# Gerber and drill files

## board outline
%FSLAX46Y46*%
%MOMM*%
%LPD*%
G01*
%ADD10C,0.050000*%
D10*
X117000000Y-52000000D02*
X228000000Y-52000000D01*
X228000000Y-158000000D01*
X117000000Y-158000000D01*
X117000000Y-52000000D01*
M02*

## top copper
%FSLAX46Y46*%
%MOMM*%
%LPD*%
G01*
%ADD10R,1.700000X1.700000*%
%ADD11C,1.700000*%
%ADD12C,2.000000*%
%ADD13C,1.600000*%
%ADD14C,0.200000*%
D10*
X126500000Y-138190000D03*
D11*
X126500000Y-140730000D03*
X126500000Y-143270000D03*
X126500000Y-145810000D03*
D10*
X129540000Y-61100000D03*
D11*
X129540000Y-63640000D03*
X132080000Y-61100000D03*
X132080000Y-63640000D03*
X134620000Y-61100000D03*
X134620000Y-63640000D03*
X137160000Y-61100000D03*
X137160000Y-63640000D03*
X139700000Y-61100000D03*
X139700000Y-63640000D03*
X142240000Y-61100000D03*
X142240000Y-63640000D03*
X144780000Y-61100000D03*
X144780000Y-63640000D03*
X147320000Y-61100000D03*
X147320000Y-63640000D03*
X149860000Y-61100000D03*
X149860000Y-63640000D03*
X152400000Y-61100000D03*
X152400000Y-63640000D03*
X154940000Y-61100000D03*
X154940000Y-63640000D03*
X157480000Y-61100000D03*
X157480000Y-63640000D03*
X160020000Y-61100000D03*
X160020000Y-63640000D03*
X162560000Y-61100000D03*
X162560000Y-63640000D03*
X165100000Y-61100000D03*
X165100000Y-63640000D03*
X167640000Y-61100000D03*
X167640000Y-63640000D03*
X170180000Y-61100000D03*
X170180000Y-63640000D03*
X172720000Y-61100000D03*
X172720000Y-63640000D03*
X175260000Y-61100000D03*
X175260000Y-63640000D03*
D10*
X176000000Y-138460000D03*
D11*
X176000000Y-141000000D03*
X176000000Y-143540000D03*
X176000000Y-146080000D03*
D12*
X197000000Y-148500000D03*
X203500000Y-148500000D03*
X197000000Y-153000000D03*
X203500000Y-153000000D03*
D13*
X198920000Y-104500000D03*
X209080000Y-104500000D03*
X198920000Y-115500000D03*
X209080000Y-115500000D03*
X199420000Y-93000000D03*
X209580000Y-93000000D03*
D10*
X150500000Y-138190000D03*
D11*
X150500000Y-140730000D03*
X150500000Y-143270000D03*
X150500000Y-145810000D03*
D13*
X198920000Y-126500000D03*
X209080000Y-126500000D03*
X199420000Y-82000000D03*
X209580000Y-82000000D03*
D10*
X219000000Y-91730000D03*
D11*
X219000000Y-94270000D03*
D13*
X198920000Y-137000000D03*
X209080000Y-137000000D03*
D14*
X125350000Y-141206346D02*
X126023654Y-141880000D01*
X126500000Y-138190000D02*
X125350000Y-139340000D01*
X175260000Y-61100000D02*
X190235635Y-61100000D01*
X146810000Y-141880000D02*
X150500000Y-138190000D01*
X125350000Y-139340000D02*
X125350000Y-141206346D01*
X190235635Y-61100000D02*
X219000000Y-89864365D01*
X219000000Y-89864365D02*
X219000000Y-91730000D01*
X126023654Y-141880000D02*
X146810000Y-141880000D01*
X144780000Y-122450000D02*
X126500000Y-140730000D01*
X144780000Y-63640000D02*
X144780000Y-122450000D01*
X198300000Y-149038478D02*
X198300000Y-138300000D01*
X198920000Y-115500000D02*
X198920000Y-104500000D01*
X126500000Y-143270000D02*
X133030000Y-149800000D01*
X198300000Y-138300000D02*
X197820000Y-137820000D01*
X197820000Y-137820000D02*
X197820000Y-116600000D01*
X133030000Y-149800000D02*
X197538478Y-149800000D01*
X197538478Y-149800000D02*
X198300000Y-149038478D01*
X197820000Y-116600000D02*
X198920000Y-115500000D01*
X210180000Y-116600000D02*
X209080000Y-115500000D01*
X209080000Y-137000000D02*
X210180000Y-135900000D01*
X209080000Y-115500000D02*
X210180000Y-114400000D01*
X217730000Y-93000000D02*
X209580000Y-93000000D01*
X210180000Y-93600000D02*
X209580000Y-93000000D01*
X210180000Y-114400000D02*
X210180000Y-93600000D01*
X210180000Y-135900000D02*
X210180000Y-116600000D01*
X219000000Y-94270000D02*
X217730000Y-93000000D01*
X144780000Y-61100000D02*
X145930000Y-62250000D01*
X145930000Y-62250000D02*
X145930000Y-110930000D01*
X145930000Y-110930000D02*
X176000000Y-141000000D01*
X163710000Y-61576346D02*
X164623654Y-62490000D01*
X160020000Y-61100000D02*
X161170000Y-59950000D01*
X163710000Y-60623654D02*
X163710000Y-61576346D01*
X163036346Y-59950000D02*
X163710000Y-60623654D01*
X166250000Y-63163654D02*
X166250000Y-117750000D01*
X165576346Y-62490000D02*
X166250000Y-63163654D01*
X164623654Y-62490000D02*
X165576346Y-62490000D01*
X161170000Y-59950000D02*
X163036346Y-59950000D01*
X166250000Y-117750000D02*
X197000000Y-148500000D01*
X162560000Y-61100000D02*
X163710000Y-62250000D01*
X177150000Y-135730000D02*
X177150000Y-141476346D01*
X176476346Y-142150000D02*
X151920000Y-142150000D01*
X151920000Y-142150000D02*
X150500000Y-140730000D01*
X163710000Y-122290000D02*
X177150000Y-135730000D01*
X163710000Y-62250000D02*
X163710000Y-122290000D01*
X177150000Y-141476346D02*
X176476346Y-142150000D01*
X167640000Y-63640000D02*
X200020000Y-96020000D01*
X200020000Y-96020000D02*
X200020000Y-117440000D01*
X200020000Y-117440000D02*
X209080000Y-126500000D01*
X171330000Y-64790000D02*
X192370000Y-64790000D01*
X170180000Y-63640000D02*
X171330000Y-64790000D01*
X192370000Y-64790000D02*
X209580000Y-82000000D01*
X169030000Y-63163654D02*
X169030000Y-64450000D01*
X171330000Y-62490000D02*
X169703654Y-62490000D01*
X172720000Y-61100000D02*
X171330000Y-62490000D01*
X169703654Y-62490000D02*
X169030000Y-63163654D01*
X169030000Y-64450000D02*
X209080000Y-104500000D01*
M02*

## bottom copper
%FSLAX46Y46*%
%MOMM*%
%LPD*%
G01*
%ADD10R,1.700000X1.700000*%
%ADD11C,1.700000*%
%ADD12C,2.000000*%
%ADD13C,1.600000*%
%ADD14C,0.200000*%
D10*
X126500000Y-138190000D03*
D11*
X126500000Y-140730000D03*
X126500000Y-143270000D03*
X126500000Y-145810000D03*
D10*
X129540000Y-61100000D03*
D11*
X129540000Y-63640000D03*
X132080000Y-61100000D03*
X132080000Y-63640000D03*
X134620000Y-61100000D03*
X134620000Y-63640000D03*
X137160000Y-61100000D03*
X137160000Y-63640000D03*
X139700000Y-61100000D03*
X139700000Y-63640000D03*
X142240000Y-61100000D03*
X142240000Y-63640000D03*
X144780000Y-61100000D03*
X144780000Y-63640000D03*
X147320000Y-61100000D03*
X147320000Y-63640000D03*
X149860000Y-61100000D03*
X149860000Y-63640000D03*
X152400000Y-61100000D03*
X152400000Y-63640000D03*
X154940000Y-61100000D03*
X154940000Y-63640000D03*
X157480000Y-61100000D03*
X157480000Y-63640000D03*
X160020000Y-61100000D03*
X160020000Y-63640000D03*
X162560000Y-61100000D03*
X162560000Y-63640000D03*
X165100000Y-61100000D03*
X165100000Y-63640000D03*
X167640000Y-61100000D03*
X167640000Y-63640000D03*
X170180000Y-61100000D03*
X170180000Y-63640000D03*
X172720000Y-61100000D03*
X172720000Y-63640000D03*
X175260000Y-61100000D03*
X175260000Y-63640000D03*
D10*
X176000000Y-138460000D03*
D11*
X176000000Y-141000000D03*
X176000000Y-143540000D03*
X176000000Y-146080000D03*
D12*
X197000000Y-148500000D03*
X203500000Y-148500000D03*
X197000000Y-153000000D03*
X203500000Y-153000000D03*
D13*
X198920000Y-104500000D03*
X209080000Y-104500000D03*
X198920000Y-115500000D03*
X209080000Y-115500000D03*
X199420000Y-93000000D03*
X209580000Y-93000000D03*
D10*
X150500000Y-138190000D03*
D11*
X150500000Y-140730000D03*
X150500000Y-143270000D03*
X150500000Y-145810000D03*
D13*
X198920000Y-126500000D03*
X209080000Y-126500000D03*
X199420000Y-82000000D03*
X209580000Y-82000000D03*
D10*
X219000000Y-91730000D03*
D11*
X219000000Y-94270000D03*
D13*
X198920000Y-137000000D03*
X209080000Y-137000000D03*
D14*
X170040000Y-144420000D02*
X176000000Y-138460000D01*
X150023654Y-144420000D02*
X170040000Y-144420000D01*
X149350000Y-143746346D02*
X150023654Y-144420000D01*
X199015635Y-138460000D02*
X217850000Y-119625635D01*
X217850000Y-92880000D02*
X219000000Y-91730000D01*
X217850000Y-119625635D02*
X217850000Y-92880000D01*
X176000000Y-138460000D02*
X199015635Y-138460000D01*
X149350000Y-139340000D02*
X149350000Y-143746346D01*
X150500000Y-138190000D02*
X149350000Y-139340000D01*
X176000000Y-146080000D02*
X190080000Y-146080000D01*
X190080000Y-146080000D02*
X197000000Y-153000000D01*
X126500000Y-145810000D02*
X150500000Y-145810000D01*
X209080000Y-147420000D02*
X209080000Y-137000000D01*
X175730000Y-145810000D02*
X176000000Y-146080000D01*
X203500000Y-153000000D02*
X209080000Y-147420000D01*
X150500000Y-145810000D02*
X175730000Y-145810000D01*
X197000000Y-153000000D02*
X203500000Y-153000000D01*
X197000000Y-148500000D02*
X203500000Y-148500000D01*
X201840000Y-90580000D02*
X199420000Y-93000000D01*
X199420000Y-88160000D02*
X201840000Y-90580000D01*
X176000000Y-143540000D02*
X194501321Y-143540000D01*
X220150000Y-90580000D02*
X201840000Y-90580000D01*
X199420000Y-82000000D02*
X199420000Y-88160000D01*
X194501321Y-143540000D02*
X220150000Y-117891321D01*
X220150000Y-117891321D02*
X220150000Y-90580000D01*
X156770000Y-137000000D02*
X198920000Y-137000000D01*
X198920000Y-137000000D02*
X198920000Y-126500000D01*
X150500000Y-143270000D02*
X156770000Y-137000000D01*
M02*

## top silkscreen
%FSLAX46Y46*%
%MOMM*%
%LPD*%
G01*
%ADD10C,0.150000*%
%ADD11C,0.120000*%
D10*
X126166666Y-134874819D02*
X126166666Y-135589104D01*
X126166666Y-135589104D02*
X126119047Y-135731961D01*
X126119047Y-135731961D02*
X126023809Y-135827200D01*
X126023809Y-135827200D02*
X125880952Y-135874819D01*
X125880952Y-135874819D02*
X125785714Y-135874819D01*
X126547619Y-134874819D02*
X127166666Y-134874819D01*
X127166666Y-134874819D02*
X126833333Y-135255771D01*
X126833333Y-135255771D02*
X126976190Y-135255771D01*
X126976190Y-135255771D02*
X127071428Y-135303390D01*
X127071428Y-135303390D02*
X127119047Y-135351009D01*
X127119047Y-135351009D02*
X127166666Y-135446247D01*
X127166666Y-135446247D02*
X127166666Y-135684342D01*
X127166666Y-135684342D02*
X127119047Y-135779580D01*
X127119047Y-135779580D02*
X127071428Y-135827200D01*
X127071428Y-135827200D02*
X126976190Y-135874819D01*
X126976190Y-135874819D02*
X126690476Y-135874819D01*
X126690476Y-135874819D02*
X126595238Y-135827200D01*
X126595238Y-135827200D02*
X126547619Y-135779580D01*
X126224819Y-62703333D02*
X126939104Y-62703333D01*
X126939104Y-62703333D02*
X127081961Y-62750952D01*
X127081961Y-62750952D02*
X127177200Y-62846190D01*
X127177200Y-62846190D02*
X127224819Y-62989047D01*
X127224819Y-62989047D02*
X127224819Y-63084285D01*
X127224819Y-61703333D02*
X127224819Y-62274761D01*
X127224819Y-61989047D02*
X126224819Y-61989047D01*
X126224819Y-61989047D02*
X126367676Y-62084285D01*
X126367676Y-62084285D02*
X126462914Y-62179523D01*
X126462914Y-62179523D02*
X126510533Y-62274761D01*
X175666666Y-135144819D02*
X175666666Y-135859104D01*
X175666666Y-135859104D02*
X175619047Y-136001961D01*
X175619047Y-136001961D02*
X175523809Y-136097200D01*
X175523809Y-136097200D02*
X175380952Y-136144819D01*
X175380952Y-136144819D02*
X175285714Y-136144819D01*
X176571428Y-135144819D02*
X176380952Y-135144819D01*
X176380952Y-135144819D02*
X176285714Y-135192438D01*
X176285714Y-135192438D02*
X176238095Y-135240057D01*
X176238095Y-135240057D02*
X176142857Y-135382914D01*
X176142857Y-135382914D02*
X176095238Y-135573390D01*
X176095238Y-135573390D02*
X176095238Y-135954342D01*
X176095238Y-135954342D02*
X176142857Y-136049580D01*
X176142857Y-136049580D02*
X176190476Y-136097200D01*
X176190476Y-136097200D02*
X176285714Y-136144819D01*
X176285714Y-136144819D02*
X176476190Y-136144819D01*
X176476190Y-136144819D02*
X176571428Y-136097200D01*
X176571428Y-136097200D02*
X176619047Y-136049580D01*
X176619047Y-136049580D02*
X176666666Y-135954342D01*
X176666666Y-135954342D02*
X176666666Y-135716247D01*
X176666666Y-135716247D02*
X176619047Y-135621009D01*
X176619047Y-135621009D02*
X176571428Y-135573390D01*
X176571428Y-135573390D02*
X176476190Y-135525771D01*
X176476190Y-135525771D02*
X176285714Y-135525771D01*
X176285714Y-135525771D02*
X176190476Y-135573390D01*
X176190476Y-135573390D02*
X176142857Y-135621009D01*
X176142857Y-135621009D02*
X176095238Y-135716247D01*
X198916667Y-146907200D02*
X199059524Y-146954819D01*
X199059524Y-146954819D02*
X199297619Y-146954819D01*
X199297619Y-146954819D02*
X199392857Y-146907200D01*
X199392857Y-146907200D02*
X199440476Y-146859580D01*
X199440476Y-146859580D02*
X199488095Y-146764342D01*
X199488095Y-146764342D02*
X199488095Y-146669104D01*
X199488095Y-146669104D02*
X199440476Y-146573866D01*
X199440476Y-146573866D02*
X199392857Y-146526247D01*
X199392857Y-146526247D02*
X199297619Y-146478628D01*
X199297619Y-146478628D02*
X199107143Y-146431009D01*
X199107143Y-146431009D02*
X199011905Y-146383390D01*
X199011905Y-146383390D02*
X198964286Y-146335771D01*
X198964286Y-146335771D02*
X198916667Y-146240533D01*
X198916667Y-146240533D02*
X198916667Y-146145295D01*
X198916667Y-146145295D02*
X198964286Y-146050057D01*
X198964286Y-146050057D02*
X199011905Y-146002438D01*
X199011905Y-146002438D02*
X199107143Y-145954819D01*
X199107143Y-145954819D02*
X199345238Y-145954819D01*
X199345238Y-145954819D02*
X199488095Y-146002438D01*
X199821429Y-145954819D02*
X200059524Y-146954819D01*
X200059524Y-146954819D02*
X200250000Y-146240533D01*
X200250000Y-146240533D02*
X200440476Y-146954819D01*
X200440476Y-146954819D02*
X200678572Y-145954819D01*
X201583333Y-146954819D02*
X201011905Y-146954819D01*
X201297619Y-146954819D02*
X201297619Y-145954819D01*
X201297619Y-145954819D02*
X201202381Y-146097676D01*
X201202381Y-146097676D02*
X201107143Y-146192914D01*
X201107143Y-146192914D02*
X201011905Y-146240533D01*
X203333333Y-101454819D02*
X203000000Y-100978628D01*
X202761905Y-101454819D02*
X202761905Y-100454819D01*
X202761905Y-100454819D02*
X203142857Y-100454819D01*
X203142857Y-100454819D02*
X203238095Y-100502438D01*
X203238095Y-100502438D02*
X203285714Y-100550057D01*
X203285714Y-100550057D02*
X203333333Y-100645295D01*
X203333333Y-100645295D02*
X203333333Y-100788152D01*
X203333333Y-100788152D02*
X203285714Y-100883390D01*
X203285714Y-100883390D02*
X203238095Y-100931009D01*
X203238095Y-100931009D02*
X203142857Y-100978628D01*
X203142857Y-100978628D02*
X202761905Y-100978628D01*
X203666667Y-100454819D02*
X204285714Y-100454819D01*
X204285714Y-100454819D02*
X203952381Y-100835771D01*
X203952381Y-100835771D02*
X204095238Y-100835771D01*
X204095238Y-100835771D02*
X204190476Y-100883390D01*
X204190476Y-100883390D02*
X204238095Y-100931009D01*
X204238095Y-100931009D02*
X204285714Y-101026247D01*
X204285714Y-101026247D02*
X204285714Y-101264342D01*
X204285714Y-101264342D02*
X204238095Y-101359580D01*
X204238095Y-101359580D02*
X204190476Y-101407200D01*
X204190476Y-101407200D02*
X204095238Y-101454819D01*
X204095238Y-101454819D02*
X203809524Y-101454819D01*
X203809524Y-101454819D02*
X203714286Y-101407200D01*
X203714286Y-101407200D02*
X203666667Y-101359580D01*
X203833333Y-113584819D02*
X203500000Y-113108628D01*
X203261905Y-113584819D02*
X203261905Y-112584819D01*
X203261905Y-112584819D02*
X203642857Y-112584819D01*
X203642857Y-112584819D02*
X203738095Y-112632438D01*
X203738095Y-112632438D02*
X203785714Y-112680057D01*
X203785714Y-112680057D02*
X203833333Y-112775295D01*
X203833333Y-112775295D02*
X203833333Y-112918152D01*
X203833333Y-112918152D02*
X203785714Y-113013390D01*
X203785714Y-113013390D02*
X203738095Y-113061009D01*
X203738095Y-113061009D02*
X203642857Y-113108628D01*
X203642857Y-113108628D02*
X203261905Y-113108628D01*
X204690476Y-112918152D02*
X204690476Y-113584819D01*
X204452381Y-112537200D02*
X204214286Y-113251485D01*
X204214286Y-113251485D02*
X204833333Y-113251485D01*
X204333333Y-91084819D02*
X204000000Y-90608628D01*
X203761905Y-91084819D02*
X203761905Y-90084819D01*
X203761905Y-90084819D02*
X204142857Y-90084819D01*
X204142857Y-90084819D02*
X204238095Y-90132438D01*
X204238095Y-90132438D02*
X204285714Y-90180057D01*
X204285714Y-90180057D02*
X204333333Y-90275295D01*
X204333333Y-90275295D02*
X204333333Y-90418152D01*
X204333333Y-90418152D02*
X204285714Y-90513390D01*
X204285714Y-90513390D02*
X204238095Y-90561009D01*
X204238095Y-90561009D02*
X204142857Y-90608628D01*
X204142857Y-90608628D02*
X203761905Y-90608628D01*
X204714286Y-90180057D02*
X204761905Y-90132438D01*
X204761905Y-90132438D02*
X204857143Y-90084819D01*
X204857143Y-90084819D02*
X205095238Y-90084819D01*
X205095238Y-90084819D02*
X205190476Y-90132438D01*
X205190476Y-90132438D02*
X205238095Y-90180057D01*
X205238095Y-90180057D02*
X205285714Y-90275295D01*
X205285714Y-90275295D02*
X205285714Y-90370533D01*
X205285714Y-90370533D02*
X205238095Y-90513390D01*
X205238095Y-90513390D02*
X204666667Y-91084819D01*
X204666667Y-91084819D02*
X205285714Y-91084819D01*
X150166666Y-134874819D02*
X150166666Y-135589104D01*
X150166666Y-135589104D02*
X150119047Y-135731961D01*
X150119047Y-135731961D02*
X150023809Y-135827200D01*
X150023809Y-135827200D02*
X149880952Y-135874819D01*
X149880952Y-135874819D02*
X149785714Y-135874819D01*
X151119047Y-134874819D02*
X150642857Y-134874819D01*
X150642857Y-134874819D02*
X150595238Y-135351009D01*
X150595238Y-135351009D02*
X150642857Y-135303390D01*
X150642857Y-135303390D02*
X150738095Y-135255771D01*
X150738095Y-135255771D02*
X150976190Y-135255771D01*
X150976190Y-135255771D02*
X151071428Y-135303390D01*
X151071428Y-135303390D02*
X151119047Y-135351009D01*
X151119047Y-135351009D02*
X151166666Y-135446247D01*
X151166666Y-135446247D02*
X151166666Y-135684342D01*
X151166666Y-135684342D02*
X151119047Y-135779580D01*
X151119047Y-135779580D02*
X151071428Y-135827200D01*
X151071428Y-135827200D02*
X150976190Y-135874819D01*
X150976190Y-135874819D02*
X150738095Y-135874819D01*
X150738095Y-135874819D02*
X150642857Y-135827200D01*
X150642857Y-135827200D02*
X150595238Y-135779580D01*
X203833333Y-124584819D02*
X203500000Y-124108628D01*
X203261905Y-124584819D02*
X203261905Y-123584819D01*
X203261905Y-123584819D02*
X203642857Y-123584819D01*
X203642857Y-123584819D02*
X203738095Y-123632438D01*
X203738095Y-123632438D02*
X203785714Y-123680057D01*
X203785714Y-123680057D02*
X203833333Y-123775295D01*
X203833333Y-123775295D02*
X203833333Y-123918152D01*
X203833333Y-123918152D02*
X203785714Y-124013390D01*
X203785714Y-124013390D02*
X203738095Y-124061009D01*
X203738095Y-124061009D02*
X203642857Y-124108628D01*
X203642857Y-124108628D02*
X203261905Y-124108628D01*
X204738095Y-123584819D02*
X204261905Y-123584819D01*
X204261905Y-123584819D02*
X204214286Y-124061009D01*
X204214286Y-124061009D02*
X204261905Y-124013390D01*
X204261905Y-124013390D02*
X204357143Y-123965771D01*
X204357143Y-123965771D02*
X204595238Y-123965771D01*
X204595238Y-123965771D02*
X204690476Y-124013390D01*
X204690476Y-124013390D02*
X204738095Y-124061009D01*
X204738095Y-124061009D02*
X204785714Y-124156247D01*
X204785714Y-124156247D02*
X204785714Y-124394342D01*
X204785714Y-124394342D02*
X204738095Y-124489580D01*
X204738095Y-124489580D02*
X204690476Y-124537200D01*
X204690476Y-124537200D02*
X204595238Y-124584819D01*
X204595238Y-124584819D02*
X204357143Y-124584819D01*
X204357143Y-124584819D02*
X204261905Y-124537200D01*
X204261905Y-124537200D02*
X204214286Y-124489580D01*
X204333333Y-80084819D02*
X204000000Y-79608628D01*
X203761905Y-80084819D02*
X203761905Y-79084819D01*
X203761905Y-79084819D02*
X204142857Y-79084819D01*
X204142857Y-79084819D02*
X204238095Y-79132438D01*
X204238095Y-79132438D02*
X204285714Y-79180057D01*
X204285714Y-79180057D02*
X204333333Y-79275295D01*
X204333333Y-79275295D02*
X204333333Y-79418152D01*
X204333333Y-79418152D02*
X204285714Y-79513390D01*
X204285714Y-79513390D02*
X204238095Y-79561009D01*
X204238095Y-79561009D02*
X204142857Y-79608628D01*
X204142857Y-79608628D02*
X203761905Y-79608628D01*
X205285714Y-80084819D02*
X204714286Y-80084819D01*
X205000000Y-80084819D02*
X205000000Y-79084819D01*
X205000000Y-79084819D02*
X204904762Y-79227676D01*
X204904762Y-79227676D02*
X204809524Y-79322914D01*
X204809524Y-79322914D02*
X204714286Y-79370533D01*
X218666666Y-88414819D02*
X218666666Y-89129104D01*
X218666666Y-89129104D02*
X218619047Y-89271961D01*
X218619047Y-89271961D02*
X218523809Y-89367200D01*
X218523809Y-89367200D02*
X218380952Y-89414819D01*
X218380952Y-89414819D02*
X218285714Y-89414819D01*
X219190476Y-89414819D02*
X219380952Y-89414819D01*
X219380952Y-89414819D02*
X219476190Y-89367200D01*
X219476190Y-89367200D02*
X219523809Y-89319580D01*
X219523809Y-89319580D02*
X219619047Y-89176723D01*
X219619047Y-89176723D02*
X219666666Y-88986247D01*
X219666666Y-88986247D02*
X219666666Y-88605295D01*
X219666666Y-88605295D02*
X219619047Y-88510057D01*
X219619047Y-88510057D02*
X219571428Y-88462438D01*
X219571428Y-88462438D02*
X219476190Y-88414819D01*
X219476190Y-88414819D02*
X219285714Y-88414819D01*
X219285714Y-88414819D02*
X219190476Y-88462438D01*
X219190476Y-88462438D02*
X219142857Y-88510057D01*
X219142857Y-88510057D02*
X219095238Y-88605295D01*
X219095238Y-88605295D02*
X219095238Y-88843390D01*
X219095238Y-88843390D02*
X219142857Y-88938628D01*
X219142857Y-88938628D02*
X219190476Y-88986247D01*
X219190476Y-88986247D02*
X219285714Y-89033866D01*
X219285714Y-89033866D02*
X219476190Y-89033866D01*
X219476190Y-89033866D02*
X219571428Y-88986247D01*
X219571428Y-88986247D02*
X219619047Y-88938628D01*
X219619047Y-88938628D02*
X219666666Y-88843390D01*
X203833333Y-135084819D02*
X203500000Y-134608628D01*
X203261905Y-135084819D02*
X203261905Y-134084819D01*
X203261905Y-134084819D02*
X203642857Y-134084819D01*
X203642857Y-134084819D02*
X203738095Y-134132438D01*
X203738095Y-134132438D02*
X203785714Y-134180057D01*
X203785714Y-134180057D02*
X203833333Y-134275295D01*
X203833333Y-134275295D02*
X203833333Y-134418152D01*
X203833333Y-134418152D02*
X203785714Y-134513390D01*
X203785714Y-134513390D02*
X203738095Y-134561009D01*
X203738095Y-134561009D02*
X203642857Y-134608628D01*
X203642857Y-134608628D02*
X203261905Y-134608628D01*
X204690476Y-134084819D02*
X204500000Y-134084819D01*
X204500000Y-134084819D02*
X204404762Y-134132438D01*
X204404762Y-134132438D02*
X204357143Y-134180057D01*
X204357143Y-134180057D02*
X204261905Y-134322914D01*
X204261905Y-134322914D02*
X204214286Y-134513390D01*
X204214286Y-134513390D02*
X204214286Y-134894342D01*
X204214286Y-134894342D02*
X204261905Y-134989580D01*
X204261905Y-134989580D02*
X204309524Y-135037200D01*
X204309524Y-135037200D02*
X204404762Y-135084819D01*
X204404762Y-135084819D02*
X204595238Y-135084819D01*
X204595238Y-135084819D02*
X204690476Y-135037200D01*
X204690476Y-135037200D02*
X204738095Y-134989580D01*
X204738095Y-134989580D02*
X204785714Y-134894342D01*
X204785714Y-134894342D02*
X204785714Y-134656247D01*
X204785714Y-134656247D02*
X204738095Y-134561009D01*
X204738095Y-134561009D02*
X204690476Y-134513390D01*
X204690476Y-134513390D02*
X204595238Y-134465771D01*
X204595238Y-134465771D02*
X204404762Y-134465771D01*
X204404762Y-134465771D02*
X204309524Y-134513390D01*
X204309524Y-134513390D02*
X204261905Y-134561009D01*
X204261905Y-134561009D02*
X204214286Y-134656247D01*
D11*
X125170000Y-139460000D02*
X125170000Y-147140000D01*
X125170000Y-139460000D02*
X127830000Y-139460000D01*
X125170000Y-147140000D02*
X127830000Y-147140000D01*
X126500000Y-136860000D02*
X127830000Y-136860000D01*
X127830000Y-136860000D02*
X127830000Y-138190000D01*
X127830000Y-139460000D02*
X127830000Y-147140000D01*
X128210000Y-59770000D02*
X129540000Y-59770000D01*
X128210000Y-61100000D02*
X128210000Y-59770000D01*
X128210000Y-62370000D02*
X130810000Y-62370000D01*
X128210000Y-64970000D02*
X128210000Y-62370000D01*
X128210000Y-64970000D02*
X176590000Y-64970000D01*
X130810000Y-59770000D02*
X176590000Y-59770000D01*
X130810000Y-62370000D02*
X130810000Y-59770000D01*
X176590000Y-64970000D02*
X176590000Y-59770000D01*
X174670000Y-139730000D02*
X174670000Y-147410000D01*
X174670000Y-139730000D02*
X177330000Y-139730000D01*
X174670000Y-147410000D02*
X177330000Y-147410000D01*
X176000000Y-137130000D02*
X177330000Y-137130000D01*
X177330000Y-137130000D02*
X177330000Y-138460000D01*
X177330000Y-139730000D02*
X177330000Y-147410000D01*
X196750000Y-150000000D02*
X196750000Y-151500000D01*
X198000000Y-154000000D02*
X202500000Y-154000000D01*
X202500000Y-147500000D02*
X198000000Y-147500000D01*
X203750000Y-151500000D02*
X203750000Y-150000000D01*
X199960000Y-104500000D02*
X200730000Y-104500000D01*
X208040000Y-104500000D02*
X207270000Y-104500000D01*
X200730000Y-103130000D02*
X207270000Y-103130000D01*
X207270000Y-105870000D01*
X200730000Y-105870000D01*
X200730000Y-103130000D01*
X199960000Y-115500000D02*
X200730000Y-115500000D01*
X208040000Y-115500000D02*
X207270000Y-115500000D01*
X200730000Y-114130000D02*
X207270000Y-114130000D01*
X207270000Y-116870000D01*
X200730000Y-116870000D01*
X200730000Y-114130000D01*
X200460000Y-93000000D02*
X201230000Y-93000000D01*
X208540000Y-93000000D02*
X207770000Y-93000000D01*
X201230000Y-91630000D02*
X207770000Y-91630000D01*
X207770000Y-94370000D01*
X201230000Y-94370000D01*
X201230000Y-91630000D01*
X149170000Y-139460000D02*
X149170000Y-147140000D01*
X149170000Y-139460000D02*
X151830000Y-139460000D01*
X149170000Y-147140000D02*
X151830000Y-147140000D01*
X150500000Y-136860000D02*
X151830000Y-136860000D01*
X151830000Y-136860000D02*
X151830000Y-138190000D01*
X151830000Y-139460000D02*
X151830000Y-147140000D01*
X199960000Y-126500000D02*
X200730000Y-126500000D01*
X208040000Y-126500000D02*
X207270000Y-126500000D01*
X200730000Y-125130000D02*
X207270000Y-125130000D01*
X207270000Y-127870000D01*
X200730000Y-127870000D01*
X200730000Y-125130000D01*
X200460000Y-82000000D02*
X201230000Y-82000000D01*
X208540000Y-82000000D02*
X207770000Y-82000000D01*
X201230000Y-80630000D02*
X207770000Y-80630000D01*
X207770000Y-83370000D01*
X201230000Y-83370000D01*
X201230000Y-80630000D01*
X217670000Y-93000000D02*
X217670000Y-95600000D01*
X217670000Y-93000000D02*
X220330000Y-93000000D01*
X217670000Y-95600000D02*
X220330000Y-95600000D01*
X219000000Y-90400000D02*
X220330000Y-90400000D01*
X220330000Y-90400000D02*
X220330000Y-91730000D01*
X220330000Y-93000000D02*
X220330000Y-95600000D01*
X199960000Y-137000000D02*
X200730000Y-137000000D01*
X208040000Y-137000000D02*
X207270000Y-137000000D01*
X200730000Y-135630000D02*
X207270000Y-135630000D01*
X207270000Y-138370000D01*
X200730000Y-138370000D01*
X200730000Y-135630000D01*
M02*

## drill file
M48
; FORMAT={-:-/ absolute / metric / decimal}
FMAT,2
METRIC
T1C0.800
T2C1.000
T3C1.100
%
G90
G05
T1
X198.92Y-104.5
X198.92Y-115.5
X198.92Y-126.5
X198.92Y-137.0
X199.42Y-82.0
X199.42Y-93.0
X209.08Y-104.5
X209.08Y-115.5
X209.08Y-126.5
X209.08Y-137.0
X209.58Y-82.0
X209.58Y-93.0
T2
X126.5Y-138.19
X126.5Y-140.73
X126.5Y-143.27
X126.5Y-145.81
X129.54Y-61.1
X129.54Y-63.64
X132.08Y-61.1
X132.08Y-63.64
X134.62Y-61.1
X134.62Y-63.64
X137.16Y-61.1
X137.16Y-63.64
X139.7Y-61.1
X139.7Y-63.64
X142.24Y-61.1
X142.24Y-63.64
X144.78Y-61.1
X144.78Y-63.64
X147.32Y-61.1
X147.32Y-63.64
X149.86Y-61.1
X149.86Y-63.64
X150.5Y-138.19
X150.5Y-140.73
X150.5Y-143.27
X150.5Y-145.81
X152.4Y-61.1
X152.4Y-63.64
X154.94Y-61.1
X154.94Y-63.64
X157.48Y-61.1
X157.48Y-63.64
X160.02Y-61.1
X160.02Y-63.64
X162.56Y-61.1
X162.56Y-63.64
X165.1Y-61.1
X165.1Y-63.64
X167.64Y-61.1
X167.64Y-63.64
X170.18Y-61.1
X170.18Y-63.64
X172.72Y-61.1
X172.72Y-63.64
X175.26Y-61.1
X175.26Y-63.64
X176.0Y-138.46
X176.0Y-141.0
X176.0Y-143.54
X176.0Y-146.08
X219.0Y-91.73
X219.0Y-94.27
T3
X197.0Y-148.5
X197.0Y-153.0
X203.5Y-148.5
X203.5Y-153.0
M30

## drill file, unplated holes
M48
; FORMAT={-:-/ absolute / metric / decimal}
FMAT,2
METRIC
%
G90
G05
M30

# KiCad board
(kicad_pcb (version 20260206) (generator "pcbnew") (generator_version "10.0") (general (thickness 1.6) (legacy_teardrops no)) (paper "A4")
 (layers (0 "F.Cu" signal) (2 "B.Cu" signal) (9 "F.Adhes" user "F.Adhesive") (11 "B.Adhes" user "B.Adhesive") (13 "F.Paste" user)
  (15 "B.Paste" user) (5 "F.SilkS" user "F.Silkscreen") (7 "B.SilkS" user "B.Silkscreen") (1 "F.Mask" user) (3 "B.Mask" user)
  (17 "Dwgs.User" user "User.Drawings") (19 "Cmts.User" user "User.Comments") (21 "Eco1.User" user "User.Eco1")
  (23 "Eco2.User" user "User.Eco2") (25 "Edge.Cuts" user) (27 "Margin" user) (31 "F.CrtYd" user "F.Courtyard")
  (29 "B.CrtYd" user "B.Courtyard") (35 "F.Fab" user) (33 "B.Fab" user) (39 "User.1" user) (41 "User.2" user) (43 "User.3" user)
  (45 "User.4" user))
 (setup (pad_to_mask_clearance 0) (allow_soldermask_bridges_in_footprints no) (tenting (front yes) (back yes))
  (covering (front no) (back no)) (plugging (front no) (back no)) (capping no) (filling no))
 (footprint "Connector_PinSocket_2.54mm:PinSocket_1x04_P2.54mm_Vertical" (layer "F.Cu") (at 126.5 138.19)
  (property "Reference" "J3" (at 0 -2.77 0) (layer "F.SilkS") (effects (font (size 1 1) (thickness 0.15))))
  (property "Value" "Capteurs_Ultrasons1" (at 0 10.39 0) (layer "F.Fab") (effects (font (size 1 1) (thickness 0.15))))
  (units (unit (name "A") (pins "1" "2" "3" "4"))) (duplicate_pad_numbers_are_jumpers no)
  (fp_line (start -1.33 1.27) (end -1.33 8.95) (stroke (width 0.12) (type solid)) (layer "F.SilkS"))
  (fp_line (start -1.33 1.27) (end 1.33 1.27) (stroke (width 0.12) (type solid)) (layer "F.SilkS"))
  (fp_line (start -1.33 8.95) (end 1.33 8.95) (stroke (width 0.12) (type solid)) (layer "F.SilkS"))
  (fp_line (start 0 -1.33) (end 1.33 -1.33) (stroke (width 0.12) (type solid)) (layer "F.SilkS"))
  (fp_line (start 1.33 -1.33) (end 1.33 0) (stroke (width 0.12) (type solid)) (layer "F.SilkS"))
  (fp_line (start 1.33 1.27) (end 1.33 8.95) (stroke (width 0.12) (type solid)) (layer "F.SilkS"))
  (pad "1" thru_hole rect (at 0 0) (size 1.7 1.7) (drill 1) (layers "*.Cu" "*.Mask") (remove_unused_layers no) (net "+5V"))
  (pad "2" thru_hole circle (at 0 2.54) (size 1.7 1.7) (drill 1) (layers "*.Cu" "*.Mask") (remove_unused_layers no) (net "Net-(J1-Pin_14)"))
  (pad "3" thru_hole circle (at 0 5.08) (size 1.7 1.7) (drill 1) (layers "*.Cu" "*.Mask") (remove_unused_layers no) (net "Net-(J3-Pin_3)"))
  (pad "4" thru_hole circle (at 0 7.62) (size 1.7 1.7) (drill 1) (layers "*.Cu" "*.Mask") (remove_unused_layers no) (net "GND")))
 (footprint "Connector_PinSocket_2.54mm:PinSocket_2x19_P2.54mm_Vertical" (layer "F.Cu") (at 129.54 61.1 90)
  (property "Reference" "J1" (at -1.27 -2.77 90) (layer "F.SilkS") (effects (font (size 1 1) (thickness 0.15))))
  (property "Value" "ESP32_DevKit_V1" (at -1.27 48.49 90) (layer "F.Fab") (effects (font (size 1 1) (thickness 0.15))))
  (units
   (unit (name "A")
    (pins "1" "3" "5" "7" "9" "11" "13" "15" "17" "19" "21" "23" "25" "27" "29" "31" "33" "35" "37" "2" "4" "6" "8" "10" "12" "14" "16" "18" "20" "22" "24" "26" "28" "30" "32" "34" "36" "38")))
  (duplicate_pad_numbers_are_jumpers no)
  (fp_line (start 1.33 -1.33) (end 1.33 0) (stroke (width 0.12) (type solid)) (layer "F.SilkS"))
  (fp_line (start 0 -1.33) (end 1.33 -1.33) (stroke (width 0.12) (type solid)) (layer "F.SilkS"))
  (fp_line (start -1.27 -1.33) (end -1.27 1.27) (stroke (width 0.12) (type solid)) (layer "F.SilkS"))
  (fp_line (start -3.87 -1.33) (end -1.27 -1.33) (stroke (width 0.12) (type solid)) (layer "F.SilkS"))
  (fp_line (start -3.87 -1.33) (end -3.87 47.05) (stroke (width 0.12) (type solid)) (layer "F.SilkS"))
  (fp_line (start 1.33 1.27) (end 1.33 47.05) (stroke (width 0.12) (type solid)) (layer "F.SilkS"))
  (fp_line (start -1.27 1.27) (end 1.33 1.27) (stroke (width 0.12) (type solid)) (layer "F.SilkS"))
  (fp_line (start -3.87 47.05) (end 1.33 47.05) (stroke (width 0.12) (type solid)) (layer "F.SilkS"))
  (pad "1" thru_hole rect (at 0 0 90) (size 1.7 1.7) (drill 1) (layers "*.Cu" "*.Mask") (remove_unused_layers no)
   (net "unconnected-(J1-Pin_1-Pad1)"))
  (pad "2" thru_hole circle (at -2.54 0 90) (size 1.7 1.7) (drill 1) (layers "*.Cu" "*.Mask") (remove_unused_layers no)
   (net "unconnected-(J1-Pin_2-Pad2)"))
  (pad "3" thru_hole circle (at 0 2.54 90) (size 1.7 1.7) (drill 1) (layers "*.Cu" "*.Mask") (remove_unused_layers no)
   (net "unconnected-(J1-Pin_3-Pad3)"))
  (pad "4" thru_hole circle (at -2.54 2.54 90) (size 1.7 1.7) (drill 1) (layers "*.Cu" "*.Mask") (remove_unused_layers no)
   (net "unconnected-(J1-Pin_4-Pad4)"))
  (pad "5" thru_hole circle (at 0 5.08 90) (size 1.7 1.7) (drill 1) (layers "*.Cu" "*.Mask") (remove_unused_layers no)
   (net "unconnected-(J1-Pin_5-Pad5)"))
  (pad "6" thru_hole circle (at -2.54 5.08 90) (size 1.7 1.7) (drill 1) (layers "*.Cu" "*.Mask") (remove_unused_layers no)
   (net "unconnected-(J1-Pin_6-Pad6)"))
  (pad "7" thru_hole circle (at 0 7.62 90) (size 1.7 1.7) (drill 1) (layers "*.Cu" "*.Mask") (remove_unused_layers no)
   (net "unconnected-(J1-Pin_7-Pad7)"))
  (pad "8" thru_hole circle (at -2.54 7.62 90) (size 1.7 1.7) (drill 1) (layers "*.Cu" "*.Mask") (remove_unused_layers no)
   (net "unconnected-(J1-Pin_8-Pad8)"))
  (pad "9" thru_hole circle (at 0 10.16 90) (size 1.7 1.7) (drill 1) (layers "*.Cu" "*.Mask") (remove_unused_layers no)
   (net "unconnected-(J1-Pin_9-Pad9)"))
  (pad "10" thru_hole circle (at -2.54 10.16 90) (size 1.7 1.7) (drill 1) (layers "*.Cu" "*.Mask") (remove_unused_layers no)
   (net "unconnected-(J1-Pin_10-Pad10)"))
  (pad "11" thru_hole circle (at 0 12.7 90) (size 1.7 1.7) (drill 1) (layers "*.Cu" "*.Mask") (remove_unused_layers no)
   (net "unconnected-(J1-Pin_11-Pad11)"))
  (pad "12" thru_hole circle (at -2.54 12.7 90) (size 1.7 1.7) (drill 1) (layers "*.Cu" "*.Mask") (remove_unused_layers no)
   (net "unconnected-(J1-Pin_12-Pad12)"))
  (pad "13" thru_hole circle (at 0 15.24 90) (size 1.7 1.7) (drill 1) (layers "*.Cu" "*.Mask") (remove_unused_layers no)
   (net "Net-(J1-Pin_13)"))
  (pad "14" thru_hole circle (at -2.54 15.24 90) (size 1.7 1.7) (drill 1) (layers "*.Cu" "*.Mask") (remove_unused_layers no)
   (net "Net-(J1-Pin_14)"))
  (pad "15" thru_hole circle (at 0 17.78 90) (size 1.7 1.7) (drill 1) (layers "*.Cu" "*.Mask") (remove_unused_layers no)
   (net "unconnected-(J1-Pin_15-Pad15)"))
  (pad "16" thru_hole circle (at -2.54 17.78 90) (size 1.7 1.7) (drill 1) (layers "*.Cu" "*.Mask") (remove_unused_layers no)
   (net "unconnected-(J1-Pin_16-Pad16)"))
  (pad "17" thru_hole circle (at 0 20.32 90) (size 1.7 1.7) (drill 1) (layers "*.Cu" "*.Mask") (remove_unused_layers no)
   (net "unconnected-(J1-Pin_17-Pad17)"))
  (pad "18" thru_hole circle (at -2.54 20.32 90) (size 1.7 1.7) (drill 1) (layers "*.Cu" "*.Mask") (remove_unused_layers no)
   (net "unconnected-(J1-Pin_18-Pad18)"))
  (pad "19" thru_hole circle (at 0 22.86 90) (size 1.7 1.7) (drill 1) (layers "*.Cu" "*.Mask") (remove_unused_layers no)
   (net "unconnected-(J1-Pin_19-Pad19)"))
  (pad "20" thru_hole circle (at -2.54 22.86 90) (size 1.7 1.7) (drill 1) (layers "*.Cu" "*.Mask") (remove_unused_layers no)
   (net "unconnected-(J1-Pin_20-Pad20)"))
  (pad "21" thru_hole circle (at 0 25.4 90) (size 1.7 1.7) (drill 1) (layers "*.Cu" "*.Mask") (remove_unused_layers no)
   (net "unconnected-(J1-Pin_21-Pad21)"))
  (pad "22" thru_hole circle (at -2.54 25.4 90) (size 1.7 1.7) (drill 1) (layers "*.Cu" "*.Mask") (remove_unused_layers no)
   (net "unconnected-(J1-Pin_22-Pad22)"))
  (pad "23" thru_hole circle (at 0 27.94 90) (size 1.7 1.7) (drill 1) (layers "*.Cu" "*.Mask") (remove_unused_layers no)
   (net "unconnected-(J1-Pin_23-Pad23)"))
  (pad "24" thru_hole circle (at -2.54 27.94 90) (size 1.7 1.7) (drill 1) (layers "*.Cu" "*.Mask") (remove_unused_layers no)
   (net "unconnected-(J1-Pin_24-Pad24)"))
  (pad "25" thru_hole circle (at 0 30.48 90) (size 1.7 1.7) (drill 1) (layers "*.Cu" "*.Mask") (remove_unused_layers no)
   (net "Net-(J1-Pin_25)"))
  (pad "26" thru_hole circle (at -2.54 30.48 90) (size 1.7 1.7) (drill 1) (layers "*.Cu" "*.Mask") (remove_unused_layers no)
   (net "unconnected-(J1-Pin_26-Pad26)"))
  (pad "27" thru_hole circle (at 0 33.02 90) (size 1.7 1.7) (drill 1) (layers "*.Cu" "*.Mask") (remove_unused_layers no)
   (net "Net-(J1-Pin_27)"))
  (pad "28" thru_hole circle (at -2.54 33.02 90) (size 1.7 1.7) (drill 1) (layers "*.Cu" "*.Mask") (remove_unused_layers no)
   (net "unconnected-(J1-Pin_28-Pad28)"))
  (pad "29" thru_hole circle (at 0 35.56 90) (size 1.7 1.7) (drill 1) (layers "*.Cu" "*.Mask") (remove_unused_layers no)
   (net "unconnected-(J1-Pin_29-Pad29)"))
  (pad "30" thru_hole circle (at -2.54 35.56 90) (size 1.7 1.7) (drill 1) (layers "*.Cu" "*.Mask") (remove_unused_layers no)
   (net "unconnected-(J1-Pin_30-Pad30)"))
  (pad "31" thru_hole circle (at 0 38.1 90) (size 1.7 1.7) (drill 1) (layers "*.Cu" "*.Mask") (remove_unused_layers no)
   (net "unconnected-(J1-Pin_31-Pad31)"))
  (pad "32" thru_hole circle (at -2.54 38.1 90) (size 1.7 1.7) (drill 1) (layers "*.Cu" "*.Mask") (remove_unused_layers no)
   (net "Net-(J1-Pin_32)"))
  (pad "33" thru_hole circle (at 0 40.64 90) (size 1.7 1.7) (drill 1) (layers "*.Cu" "*.Mask") (remove_unused_layers no)
   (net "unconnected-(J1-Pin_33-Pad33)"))
  (pad "34" thru_hole circle (at -2.54 40.64 90) (size 1.7 1.7) (drill 1) (layers "*.Cu" "*.Mask") (remove_unused_layers no)
   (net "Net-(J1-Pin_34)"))
  (pad "35" thru_hole circle (at 0 43.18 90) (size 1.7 1.7) (drill 1) (layers "*.Cu" "*.Mask") (remove_unused_layers no)
   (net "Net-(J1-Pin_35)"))
  (pad "36" thru_hole circle (at -2.54 43.18 90) (size 1.7 1.7) (drill 1) (layers "*.Cu" "*.Mask") (remove_unused_layers no)
   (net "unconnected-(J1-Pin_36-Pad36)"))
  (pad "37" thru_hole circle (at 0 45.72 90) (size 1.7 1.7) (drill 1) (layers "*.Cu" "*.Mask") (remove_unused_layers no) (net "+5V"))
  (pad "38" thru_hole circle (at -2.54 45.72 90) (size 1.7 1.7) (drill 1) (layers "*.Cu" "*.Mask") (remove_unused_layers no)
   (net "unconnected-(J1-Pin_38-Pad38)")))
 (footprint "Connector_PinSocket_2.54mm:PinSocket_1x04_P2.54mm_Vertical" (layer "F.Cu") (at 176 138.46)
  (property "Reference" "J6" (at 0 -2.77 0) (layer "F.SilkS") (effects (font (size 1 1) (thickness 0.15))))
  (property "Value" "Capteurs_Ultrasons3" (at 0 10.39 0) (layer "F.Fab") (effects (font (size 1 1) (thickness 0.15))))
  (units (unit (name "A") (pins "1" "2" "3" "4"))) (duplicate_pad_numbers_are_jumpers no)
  (fp_line (start -1.33 1.27) (end -1.33 8.95) (stroke (width 0.12) (type solid)) (layer "F.SilkS"))
  (fp_line (start -1.33 1.27) (end 1.33 1.27) (stroke (width 0.12) (type solid)) (layer "F.SilkS"))
  (fp_line (start -1.33 8.95) (end 1.33 8.95) (stroke (width 0.12) (type solid)) (layer "F.SilkS"))
  (fp_line (start 0 -1.33) (end 1.33 -1.33) (stroke (width 0.12) (type solid)) (layer "F.SilkS"))
  (fp_line (start 1.33 -1.33) (end 1.33 0) (stroke (width 0.12) (type solid)) (layer "F.SilkS"))
  (fp_line (start 1.33 1.27) (end 1.33 8.95) (stroke (width 0.12) (type solid)) (layer "F.SilkS"))
  (pad "1" thru_hole rect (at 0 0) (size 1.7 1.7) (drill 1) (layers "*.Cu" "*.Mask") (remove_unused_layers no) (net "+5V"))
  (pad "2" thru_hole circle (at 0 2.54) (size 1.7 1.7) (drill 1) (layers "*.Cu" "*.Mask") (remove_unused_layers no) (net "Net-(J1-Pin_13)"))
  (pad "3" thru_hole circle (at 0 5.08) (size 1.7 1.7) (drill 1) (layers "*.Cu" "*.Mask") (remove_unused_layers no) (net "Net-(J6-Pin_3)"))
  (pad "4" thru_hole circle (at 0 7.62) (size 1.7 1.7) (drill 1) (layers "*.Cu" "*.Mask") (remove_unused_layers no) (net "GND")))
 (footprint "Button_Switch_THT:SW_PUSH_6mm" (layer "F.Cu") (at 197 148.5)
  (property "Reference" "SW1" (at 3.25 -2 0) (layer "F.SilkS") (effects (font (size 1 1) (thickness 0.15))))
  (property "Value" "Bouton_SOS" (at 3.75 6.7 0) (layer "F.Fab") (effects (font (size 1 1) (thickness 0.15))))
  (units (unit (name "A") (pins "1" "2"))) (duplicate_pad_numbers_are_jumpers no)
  (fp_line (start -0.25 1.5) (end -0.25 3) (stroke (width 0.12) (type solid)) (layer "F.SilkS"))
  (fp_line (start 1 5.5) (end 5.5 5.5) (stroke (width 0.12) (type solid)) (layer "F.SilkS"))
  (fp_line (start 5.5 -1) (end 1 -1) (stroke (width 0.12) (type solid)) (layer "F.SilkS"))
  (fp_line (start 6.75 3) (end 6.75 1.5) (stroke (width 0.12) (type solid)) (layer "F.SilkS"))
  (pad "1" thru_hole circle (at 0 0 90) (size 2 2) (drill 1.1) (layers "*.Cu" "*.Mask") (remove_unused_layers no) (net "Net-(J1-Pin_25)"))
  (pad "1" thru_hole circle (at 6.5 0 90) (size 2 2) (drill 1.1) (layers "*.Cu" "*.Mask") (remove_unused_layers no) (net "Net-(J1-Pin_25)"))
  (pad "2" thru_hole circle (at 0 4.5 90) (size 2 2) (drill 1.1) (layers "*.Cu" "*.Mask") (remove_unused_layers no) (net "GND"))
  (pad "2" thru_hole circle (at 6.5 4.5 90) (size 2 2) (drill 1.1) (layers "*.Cu" "*.Mask") (remove_unused_layers no) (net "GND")))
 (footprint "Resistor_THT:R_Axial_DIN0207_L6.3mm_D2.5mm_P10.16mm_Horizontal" (layer "F.Cu") (at 198.92 104.5)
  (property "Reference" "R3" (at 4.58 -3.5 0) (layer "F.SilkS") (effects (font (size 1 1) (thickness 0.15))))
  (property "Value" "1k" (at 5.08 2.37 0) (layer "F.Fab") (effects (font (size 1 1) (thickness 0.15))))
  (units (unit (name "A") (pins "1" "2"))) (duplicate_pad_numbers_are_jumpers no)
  (fp_line (start 1.04 0) (end 1.81 0) (stroke (width 0.12) (type solid)) (layer "F.SilkS"))
  (fp_line (start 9.12 0) (end 8.35 0) (stroke (width 0.12) (type solid)) (layer "F.SilkS"))
  (fp_rect (start 1.81 -1.37) (end 8.35 1.37) (stroke (width 0.12) (type solid)) (fill no) (layer "F.SilkS"))
  (pad "1" thru_hole circle (at 0 0) (size 1.6 1.6) (drill 0.8) (layers "*.Cu" "*.Mask") (remove_unused_layers no) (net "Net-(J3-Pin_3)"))
  (pad "2" thru_hole circle (at 10.16 0) (size 1.6 1.6) (drill 0.8) (layers "*.Cu" "*.Mask") (remove_unused_layers no)
   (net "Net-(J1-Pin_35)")))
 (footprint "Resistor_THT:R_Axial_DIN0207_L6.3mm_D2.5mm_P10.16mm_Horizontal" (layer "F.Cu") (at 198.92 115.5)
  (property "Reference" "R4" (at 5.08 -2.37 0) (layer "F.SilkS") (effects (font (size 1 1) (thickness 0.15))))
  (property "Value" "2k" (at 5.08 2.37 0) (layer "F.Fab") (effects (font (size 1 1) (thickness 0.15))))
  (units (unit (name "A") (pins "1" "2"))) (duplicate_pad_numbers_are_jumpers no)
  (fp_line (start 1.04 0) (end 1.81 0) (stroke (width 0.12) (type solid)) (layer "F.SilkS"))
  (fp_line (start 9.12 0) (end 8.35 0) (stroke (width 0.12) (type solid)) (layer "F.SilkS"))
  (fp_rect (start 1.81 -1.37) (end 8.35 1.37) (stroke (width 0.12) (type solid)) (fill no) (layer "F.SilkS"))
  (pad "1" thru_hole circle (at 0 0) (size 1.6 1.6) (drill 0.8) (layers "*.Cu" "*.Mask") (remove_unused_layers no) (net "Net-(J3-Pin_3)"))
  (pad "2" thru_hole circle (at 10.16 0) (size 1.6 1.6) (drill 0.8) (layers "*.Cu" "*.Mask") (remove_unused_layers no) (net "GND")))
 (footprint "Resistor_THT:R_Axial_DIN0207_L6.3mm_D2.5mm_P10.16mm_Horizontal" (layer "F.Cu") (at 199.42 93)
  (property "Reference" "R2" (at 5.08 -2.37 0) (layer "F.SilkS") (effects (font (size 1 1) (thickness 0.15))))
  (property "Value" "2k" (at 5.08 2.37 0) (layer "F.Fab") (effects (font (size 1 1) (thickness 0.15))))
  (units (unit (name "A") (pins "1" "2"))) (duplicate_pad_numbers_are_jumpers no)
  (fp_line (start 1.04 0) (end 1.81 0) (stroke (width 0.12) (type solid)) (layer "F.SilkS"))
  (fp_line (start 9.12 0) (end 8.35 0) (stroke (width 0.12) (type solid)) (layer "F.SilkS"))
  (fp_rect (start 1.81 -1.37) (end 8.35 1.37) (stroke (width 0.12) (type solid)) (fill no) (layer "F.SilkS"))
  (pad "1" thru_hole circle (at 0 0) (size 1.6 1.6) (drill 0.8) (layers "*.Cu" "*.Mask") (remove_unused_layers no) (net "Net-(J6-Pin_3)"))
  (pad "2" thru_hole circle (at 10.16 0) (size 1.6 1.6) (drill 0.8) (layers "*.Cu" "*.Mask") (remove_unused_layers no) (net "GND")))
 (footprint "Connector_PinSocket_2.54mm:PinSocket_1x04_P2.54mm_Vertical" (layer "F.Cu") (at 150.5 138.19)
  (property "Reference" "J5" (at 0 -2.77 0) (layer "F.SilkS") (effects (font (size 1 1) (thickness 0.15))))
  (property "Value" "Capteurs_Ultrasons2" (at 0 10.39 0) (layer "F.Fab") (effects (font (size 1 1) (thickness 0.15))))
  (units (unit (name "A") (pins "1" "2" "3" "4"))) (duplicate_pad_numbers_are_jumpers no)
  (fp_line (start -1.33 1.27) (end -1.33 8.95) (stroke (width 0.12) (type solid)) (layer "F.SilkS"))
  (fp_line (start -1.33 1.27) (end 1.33 1.27) (stroke (width 0.12) (type solid)) (layer "F.SilkS"))
  (fp_line (start -1.33 8.95) (end 1.33 8.95) (stroke (width 0.12) (type solid)) (layer "F.SilkS"))
  (fp_line (start 0 -1.33) (end 1.33 -1.33) (stroke (width 0.12) (type solid)) (layer "F.SilkS"))
  (fp_line (start 1.33 -1.33) (end 1.33 0) (stroke (width 0.12) (type solid)) (layer "F.SilkS"))
  (fp_line (start 1.33 1.27) (end 1.33 8.95) (stroke (width 0.12) (type solid)) (layer "F.SilkS"))
  (pad "1" thru_hole rect (at 0 0) (size 1.7 1.7) (drill 1) (layers "*.Cu" "*.Mask") (remove_unused_layers no) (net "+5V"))
  (pad "2" thru_hole circle (at 0 2.54) (size 1.7 1.7) (drill 1) (layers "*.Cu" "*.Mask") (remove_unused_layers no) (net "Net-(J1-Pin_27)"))
  (pad "3" thru_hole circle (at 0 5.08) (size 1.7 1.7) (drill 1) (layers "*.Cu" "*.Mask") (remove_unused_layers no) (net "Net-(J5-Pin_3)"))
  (pad "4" thru_hole circle (at 0 7.62) (size 1.7 1.7) (drill 1) (layers "*.Cu" "*.Mask") (remove_unused_layers no) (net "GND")))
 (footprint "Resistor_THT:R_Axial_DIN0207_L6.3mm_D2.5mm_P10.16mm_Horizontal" (layer "F.Cu") (at 198.92 126.5)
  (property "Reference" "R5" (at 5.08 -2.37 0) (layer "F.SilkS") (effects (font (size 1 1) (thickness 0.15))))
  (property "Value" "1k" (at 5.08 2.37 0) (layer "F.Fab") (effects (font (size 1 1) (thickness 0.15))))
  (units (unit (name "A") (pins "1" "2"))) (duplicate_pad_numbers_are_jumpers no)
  (fp_line (start 1.04 0) (end 1.81 0) (stroke (width 0.12) (type solid)) (layer "F.SilkS"))
  (fp_line (start 9.12 0) (end 8.35 0) (stroke (width 0.12) (type solid)) (layer "F.SilkS"))
  (fp_rect (start 1.81 -1.37) (end 8.35 1.37) (stroke (width 0.12) (type solid)) (fill no) (layer "F.SilkS"))
  (pad "1" thru_hole circle (at 0 0) (size 1.6 1.6) (drill 0.8) (layers "*.Cu" "*.Mask") (remove_unused_layers no) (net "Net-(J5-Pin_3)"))
  (pad "2" thru_hole circle (at 10.16 0) (size 1.6 1.6) (drill 0.8) (layers "*.Cu" "*.Mask") (remove_unused_layers no)
   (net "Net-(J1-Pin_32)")))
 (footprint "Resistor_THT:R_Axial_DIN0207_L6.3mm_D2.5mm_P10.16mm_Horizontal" (layer "F.Cu") (at 199.42 82)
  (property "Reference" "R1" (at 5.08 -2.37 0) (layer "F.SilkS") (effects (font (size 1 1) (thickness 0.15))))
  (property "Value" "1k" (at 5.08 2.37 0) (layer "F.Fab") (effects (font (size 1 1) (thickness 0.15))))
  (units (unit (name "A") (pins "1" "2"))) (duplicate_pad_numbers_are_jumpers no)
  (fp_line (start 1.04 0) (end 1.81 0) (stroke (width 0.12) (type solid)) (layer "F.SilkS"))
  (fp_line (start 9.12 0) (end 8.35 0) (stroke (width 0.12) (type solid)) (layer "F.SilkS"))
  (fp_rect (start 1.81 -1.37) (end 8.35 1.37) (stroke (width 0.12) (type solid)) (fill no) (layer "F.SilkS"))
  (pad "1" thru_hole circle (at 0 0) (size 1.6 1.6) (drill 0.8) (layers "*.Cu" "*.Mask") (remove_unused_layers no) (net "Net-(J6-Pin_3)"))
  (pad "2" thru_hole circle (at 10.16 0) (size 1.6 1.6) (drill 0.8) (layers "*.Cu" "*.Mask") (remove_unused_layers no)
   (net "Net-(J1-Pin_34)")))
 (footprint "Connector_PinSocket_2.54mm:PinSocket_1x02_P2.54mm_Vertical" (layer "F.Cu") (at 219 91.73)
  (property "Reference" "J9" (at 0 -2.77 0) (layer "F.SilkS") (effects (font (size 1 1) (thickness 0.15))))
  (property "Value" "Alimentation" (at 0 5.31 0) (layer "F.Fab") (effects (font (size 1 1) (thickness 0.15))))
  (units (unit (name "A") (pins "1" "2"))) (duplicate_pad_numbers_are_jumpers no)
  (fp_line (start -1.33 1.27) (end -1.33 3.87) (stroke (width 0.12) (type solid)) (layer "F.SilkS"))
  (fp_line (start -1.33 1.27) (end 1.33 1.27) (stroke (width 0.12) (type solid)) (layer "F.SilkS"))
  (fp_line (start -1.33 3.87) (end 1.33 3.87) (stroke (width 0.12) (type solid)) (layer "F.SilkS"))
  (fp_line (start 0 -1.33) (end 1.33 -1.33) (stroke (width 0.12) (type solid)) (layer "F.SilkS"))
  (fp_line (start 1.33 -1.33) (end 1.33 0) (stroke (width 0.12) (type solid)) (layer "F.SilkS"))
  (fp_line (start 1.33 1.27) (end 1.33 3.87) (stroke (width 0.12) (type solid)) (layer "F.SilkS"))
  (pad "1" thru_hole rect (at 0 0) (size 1.7 1.7) (drill 1) (layers "*.Cu" "*.Mask") (remove_unused_layers no) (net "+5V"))
  (pad "2" thru_hole circle (at 0 2.54) (size 1.7 1.7) (drill 1) (layers "*.Cu" "*.Mask") (remove_unused_layers no) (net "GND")))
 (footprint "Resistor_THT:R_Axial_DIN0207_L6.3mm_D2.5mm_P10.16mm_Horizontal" (layer "F.Cu") (at 198.92 137)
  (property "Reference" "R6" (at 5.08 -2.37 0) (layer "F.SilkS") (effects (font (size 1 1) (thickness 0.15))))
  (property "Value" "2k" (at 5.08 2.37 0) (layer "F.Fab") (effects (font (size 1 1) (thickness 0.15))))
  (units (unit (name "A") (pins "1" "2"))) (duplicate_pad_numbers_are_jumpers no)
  (fp_line (start 1.04 0) (end 1.81 0) (stroke (width 0.12) (type solid)) (layer "F.SilkS"))
  (fp_line (start 9.12 0) (end 8.35 0) (stroke (width 0.12) (type solid)) (layer "F.SilkS"))
  (fp_rect (start 1.81 -1.37) (end 8.35 1.37) (stroke (width 0.12) (type solid)) (fill no) (layer "F.SilkS"))
  (pad "1" thru_hole circle (at 0 0) (size 1.6 1.6) (drill 0.8) (layers "*.Cu" "*.Mask") (remove_unused_layers no) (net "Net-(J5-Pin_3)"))
  (pad "2" thru_hole circle (at 10.16 0) (size 1.6 1.6) (drill 0.8) (layers "*.Cu" "*.Mask") (remove_unused_layers no) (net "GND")))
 (gr_rect (start 117 52) (end 228 158) (stroke (width 0.05) (type default)) (fill no) (layer "Edge.Cuts"))
 (segment (start 125.35 141.206346) (end 126.023654 141.88) (width 0.2) (layer "F.Cu") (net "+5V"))
 (segment (start 126.5 138.19) (end 125.35 139.34) (width 0.2) (layer "F.Cu") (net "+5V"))
 (segment (start 175.26 61.1) (end 190.235635 61.1) (width 0.2) (layer "F.Cu") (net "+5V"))
 (segment (start 146.81 141.88) (end 150.5 138.19) (width 0.2) (layer "F.Cu") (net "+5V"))
 (segment (start 125.35 139.34) (end 125.35 141.206346) (width 0.2) (layer "F.Cu") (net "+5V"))
 (segment (start 190.235635 61.1) (end 219 89.864365) (width 0.2) (layer "F.Cu") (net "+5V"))
 (segment (start 219 89.864365) (end 219 91.73) (width 0.2) (layer "F.Cu") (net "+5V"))
 (segment (start 126.023654 141.88) (end 146.81 141.88) (width 0.2) (layer "F.Cu") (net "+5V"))
 (segment (start 170.04 144.42) (end 176 138.46) (width 0.2) (layer "B.Cu") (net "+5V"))
 (segment (start 150.023654 144.42) (end 170.04 144.42) (width 0.2) (layer "B.Cu") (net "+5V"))
 (segment (start 149.35 143.746346) (end 150.023654 144.42) (width 0.2) (layer "B.Cu") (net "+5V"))
 (segment (start 199.015635 138.46) (end 217.85 119.625635) (width 0.2) (layer "B.Cu") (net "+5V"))
 (segment (start 217.85 92.88) (end 219 91.73) (width 0.2) (layer "B.Cu") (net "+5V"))
 (segment (start 217.85 119.625635) (end 217.85 92.88) (width 0.2) (layer "B.Cu") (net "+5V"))
 (segment (start 176 138.46) (end 199.015635 138.46) (width 0.2) (layer "B.Cu") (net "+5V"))
 (segment (start 149.35 139.34) (end 149.35 143.746346) (width 0.2) (layer "B.Cu") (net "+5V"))
 (segment (start 150.5 138.19) (end 149.35 139.34) (width 0.2) (layer "B.Cu") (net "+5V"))
 (segment (start 144.78 122.45) (end 126.5 140.73) (width 0.2) (layer "F.Cu") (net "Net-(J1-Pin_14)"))
 (segment (start 144.78 63.64) (end 144.78 122.45) (width 0.2) (layer "F.Cu") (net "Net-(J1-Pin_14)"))
 (segment (start 198.3 149.038478) (end 198.3 138.3) (width 0.2) (layer "F.Cu") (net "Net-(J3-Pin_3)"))
 (segment (start 198.92 115.5) (end 198.92 104.5) (width 0.2) (layer "F.Cu") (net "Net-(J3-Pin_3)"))
 (segment (start 126.5 143.27) (end 133.03 149.8) (width 0.2) (layer "F.Cu") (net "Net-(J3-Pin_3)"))
 (segment (start 198.3 138.3) (end 197.82 137.82) (width 0.2) (layer "F.Cu") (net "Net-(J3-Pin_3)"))
 (segment (start 197.82 137.82) (end 197.82 116.6) (width 0.2) (layer "F.Cu") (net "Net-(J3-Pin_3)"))
 (segment (start 133.03 149.8) (end 197.538478 149.8) (width 0.2) (layer "F.Cu") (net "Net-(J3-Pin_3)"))
 (segment (start 197.538478 149.8) (end 198.3 149.038478) (width 0.2) (layer "F.Cu") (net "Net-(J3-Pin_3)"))
 (segment (start 197.82 116.6) (end 198.92 115.5) (width 0.2) (layer "F.Cu") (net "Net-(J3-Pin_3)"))
 (segment (start 210.18 116.6) (end 209.08 115.5) (width 0.2) (layer "F.Cu") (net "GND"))
 (segment (start 209.08 137) (end 210.18 135.9) (width 0.2) (layer "F.Cu") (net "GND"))
 (segment (start 209.08 115.5) (end 210.18 114.4) (width 0.2) (layer "F.Cu") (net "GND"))
 (segment (start 217.73 93) (end 209.58 93) (width 0.2) (layer "F.Cu") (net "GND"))
 (segment (start 210.18 93.6) (end 209.58 93) (width 0.2) (layer "F.Cu") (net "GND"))
 (segment (start 210.18 114.4) (end 210.18 93.6) (width 0.2) (layer "F.Cu") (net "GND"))
 (segment (start 210.18 135.9) (end 210.18 116.6) (width 0.2) (layer "F.Cu") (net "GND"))
 (segment (start 219 94.27) (end 217.73 93) (width 0.2) (layer "F.Cu") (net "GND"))
 (segment (start 176 146.08) (end 190.08 146.08) (width 0.2) (layer "B.Cu") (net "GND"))
 (segment (start 190.08 146.08) (end 197 153) (width 0.2) (layer "B.Cu") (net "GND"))
 (segment (start 126.5 145.81) (end 150.5 145.81) (width 0.2) (layer "B.Cu") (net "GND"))
 (segment (start 209.08 147.42) (end 209.08 137) (width 0.2) (layer "B.Cu") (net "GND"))
 (segment (start 175.73 145.81) (end 176 146.08) (width 0.2) (layer "B.Cu") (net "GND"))
 (segment (start 203.5 153) (end 209.08 147.42) (width 0.2) (layer "B.Cu") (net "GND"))
 (segment (start 150.5 145.81) (end 175.73 145.81) (width 0.2) (layer "B.Cu") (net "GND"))
 (segment (start 197 153) (end 203.5 153) (width 0.2) (layer "B.Cu") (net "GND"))
 (segment (start 144.78 61.1) (end 145.93 62.25) (width 0.2) (layer "F.Cu") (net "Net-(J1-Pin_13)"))
 (segment (start 145.93 62.25) (end 145.93 110.93) (width 0.2) (layer "F.Cu") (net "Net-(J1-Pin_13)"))
 (segment (start 145.93 110.93) (end 176 141) (width 0.2) (layer "F.Cu") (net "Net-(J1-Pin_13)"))
 (segment (start 163.71 61.576346) (end 164.623654 62.49) (width 0.2) (layer "F.Cu") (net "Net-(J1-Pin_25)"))
 (segment (start 160.02 61.1) (end 161.17 59.95) (width 0.2) (layer "F.Cu") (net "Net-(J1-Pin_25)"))
 (segment (start 163.71 60.623654) (end 163.71 61.576346) (width 0.2) (layer "F.Cu") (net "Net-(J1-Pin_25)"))
 (segment (start 163.036346 59.95) (end 163.71 60.623654) (width 0.2) (layer "F.Cu") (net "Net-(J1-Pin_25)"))
 (segment (start 166.25 63.163654) (end 166.25 117.75) (width 0.2) (layer "F.Cu") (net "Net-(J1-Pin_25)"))
 (segment (start 165.576346 62.49) (end 166.25 63.163654) (width 0.2) (layer "F.Cu") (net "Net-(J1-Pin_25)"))
 (segment (start 164.623654 62.49) (end 165.576346 62.49) (width 0.2) (layer "F.Cu") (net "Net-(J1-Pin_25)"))
 (segment (start 161.17 59.95) (end 163.036346 59.95) (width 0.2) (layer "F.Cu") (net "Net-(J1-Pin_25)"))
 (segment (start 166.25 117.75) (end 197 148.5) (width 0.2) (layer "F.Cu") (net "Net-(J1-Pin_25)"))
 (segment (start 197 148.5) (end 203.5 148.5) (width 0.2) (layer "B.Cu") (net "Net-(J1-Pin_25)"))
 (segment (start 162.56 61.1) (end 163.71 62.25) (width 0.2) (layer "F.Cu") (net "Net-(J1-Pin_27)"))
 (segment (start 177.15 135.73) (end 177.15 141.476346) (width 0.2) (layer "F.Cu") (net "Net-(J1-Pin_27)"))
 (segment (start 176.476346 142.15) (end 151.92 142.15) (width 0.2) (layer "F.Cu") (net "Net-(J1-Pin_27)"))
 (segment (start 151.92 142.15) (end 150.5 140.73) (width 0.2) (layer "F.Cu") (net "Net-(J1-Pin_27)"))
 (segment (start 163.71 122.29) (end 177.15 135.73) (width 0.2) (layer "F.Cu") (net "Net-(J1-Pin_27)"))
 (segment (start 163.71 62.25) (end 163.71 122.29) (width 0.2) (layer "F.Cu") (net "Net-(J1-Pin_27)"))
 (segment (start 177.15 141.476346) (end 176.476346 142.15) (width 0.2) (layer "F.Cu") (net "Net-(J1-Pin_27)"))
 (segment (start 167.64 63.64) (end 200.02 96.02) (width 0.2) (layer "F.Cu") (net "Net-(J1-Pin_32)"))
 (segment (start 200.02 96.02) (end 200.02 117.44) (width 0.2) (layer "F.Cu") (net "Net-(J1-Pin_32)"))
 (segment (start 200.02 117.44) (end 209.08 126.5) (width 0.2) (layer "F.Cu") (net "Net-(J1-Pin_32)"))
 (segment (start 171.33 64.79) (end 192.37 64.79) (width 0.2) (layer "F.Cu") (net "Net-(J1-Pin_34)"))
 (segment (start 170.18 63.64) (end 171.33 64.79) (width 0.2) (layer "F.Cu") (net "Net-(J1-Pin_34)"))
 (segment (start 192.37 64.79) (end 209.58 82) (width 0.2) (layer "F.Cu") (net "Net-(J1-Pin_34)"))
 (segment (start 169.03 63.163654) (end 169.03 64.45) (width 0.2) (layer "F.Cu") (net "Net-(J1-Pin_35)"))
 (segment (start 171.33 62.49) (end 169.703654 62.49) (width 0.2) (layer "F.Cu") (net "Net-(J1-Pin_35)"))
 (segment (start 172.72 61.1) (end 171.33 62.49) (width 0.2) (layer "F.Cu") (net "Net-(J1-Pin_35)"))
 (segment (start 169.703654 62.49) (end 169.03 63.163654) (width 0.2) (layer "F.Cu") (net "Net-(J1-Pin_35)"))
 (segment (start 169.03 64.45) (end 209.08 104.5) (width 0.2) (layer "F.Cu") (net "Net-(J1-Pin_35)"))
 (segment (start 201.84 90.58) (end 199.42 93) (width 0.2) (layer "B.Cu") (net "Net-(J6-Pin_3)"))
 (segment (start 199.42 88.16) (end 201.84 90.58) (width 0.2) (layer "B.Cu") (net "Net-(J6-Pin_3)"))
 (segment (start 176 143.54) (end 194.501321 143.54) (width 0.2) (layer "B.Cu") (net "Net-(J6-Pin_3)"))
 (segment (start 220.15 90.58) (end 201.84 90.58) (width 0.2) (layer "B.Cu") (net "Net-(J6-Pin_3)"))
 (segment (start 199.42 82) (end 199.42 88.16) (width 0.2) (layer "B.Cu") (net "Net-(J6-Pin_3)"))
 (segment (start 194.501321 143.54) (end 220.15 117.891321) (width 0.2) (layer "B.Cu") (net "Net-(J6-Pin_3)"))
 (segment (start 220.15 117.891321) (end 220.15 90.58) (width 0.2) (layer "B.Cu") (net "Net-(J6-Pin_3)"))
 (segment (start 156.77 137) (end 198.92 137) (width 0.2) (layer "B.Cu") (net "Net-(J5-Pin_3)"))
 (segment (start 198.92 137) (end 198.92 126.5) (width 0.2) (layer "B.Cu") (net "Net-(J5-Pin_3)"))
 (segment (start 150.5 143.27) (end 156.77 137) (width 0.2) (layer "B.Cu") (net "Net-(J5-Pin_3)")))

